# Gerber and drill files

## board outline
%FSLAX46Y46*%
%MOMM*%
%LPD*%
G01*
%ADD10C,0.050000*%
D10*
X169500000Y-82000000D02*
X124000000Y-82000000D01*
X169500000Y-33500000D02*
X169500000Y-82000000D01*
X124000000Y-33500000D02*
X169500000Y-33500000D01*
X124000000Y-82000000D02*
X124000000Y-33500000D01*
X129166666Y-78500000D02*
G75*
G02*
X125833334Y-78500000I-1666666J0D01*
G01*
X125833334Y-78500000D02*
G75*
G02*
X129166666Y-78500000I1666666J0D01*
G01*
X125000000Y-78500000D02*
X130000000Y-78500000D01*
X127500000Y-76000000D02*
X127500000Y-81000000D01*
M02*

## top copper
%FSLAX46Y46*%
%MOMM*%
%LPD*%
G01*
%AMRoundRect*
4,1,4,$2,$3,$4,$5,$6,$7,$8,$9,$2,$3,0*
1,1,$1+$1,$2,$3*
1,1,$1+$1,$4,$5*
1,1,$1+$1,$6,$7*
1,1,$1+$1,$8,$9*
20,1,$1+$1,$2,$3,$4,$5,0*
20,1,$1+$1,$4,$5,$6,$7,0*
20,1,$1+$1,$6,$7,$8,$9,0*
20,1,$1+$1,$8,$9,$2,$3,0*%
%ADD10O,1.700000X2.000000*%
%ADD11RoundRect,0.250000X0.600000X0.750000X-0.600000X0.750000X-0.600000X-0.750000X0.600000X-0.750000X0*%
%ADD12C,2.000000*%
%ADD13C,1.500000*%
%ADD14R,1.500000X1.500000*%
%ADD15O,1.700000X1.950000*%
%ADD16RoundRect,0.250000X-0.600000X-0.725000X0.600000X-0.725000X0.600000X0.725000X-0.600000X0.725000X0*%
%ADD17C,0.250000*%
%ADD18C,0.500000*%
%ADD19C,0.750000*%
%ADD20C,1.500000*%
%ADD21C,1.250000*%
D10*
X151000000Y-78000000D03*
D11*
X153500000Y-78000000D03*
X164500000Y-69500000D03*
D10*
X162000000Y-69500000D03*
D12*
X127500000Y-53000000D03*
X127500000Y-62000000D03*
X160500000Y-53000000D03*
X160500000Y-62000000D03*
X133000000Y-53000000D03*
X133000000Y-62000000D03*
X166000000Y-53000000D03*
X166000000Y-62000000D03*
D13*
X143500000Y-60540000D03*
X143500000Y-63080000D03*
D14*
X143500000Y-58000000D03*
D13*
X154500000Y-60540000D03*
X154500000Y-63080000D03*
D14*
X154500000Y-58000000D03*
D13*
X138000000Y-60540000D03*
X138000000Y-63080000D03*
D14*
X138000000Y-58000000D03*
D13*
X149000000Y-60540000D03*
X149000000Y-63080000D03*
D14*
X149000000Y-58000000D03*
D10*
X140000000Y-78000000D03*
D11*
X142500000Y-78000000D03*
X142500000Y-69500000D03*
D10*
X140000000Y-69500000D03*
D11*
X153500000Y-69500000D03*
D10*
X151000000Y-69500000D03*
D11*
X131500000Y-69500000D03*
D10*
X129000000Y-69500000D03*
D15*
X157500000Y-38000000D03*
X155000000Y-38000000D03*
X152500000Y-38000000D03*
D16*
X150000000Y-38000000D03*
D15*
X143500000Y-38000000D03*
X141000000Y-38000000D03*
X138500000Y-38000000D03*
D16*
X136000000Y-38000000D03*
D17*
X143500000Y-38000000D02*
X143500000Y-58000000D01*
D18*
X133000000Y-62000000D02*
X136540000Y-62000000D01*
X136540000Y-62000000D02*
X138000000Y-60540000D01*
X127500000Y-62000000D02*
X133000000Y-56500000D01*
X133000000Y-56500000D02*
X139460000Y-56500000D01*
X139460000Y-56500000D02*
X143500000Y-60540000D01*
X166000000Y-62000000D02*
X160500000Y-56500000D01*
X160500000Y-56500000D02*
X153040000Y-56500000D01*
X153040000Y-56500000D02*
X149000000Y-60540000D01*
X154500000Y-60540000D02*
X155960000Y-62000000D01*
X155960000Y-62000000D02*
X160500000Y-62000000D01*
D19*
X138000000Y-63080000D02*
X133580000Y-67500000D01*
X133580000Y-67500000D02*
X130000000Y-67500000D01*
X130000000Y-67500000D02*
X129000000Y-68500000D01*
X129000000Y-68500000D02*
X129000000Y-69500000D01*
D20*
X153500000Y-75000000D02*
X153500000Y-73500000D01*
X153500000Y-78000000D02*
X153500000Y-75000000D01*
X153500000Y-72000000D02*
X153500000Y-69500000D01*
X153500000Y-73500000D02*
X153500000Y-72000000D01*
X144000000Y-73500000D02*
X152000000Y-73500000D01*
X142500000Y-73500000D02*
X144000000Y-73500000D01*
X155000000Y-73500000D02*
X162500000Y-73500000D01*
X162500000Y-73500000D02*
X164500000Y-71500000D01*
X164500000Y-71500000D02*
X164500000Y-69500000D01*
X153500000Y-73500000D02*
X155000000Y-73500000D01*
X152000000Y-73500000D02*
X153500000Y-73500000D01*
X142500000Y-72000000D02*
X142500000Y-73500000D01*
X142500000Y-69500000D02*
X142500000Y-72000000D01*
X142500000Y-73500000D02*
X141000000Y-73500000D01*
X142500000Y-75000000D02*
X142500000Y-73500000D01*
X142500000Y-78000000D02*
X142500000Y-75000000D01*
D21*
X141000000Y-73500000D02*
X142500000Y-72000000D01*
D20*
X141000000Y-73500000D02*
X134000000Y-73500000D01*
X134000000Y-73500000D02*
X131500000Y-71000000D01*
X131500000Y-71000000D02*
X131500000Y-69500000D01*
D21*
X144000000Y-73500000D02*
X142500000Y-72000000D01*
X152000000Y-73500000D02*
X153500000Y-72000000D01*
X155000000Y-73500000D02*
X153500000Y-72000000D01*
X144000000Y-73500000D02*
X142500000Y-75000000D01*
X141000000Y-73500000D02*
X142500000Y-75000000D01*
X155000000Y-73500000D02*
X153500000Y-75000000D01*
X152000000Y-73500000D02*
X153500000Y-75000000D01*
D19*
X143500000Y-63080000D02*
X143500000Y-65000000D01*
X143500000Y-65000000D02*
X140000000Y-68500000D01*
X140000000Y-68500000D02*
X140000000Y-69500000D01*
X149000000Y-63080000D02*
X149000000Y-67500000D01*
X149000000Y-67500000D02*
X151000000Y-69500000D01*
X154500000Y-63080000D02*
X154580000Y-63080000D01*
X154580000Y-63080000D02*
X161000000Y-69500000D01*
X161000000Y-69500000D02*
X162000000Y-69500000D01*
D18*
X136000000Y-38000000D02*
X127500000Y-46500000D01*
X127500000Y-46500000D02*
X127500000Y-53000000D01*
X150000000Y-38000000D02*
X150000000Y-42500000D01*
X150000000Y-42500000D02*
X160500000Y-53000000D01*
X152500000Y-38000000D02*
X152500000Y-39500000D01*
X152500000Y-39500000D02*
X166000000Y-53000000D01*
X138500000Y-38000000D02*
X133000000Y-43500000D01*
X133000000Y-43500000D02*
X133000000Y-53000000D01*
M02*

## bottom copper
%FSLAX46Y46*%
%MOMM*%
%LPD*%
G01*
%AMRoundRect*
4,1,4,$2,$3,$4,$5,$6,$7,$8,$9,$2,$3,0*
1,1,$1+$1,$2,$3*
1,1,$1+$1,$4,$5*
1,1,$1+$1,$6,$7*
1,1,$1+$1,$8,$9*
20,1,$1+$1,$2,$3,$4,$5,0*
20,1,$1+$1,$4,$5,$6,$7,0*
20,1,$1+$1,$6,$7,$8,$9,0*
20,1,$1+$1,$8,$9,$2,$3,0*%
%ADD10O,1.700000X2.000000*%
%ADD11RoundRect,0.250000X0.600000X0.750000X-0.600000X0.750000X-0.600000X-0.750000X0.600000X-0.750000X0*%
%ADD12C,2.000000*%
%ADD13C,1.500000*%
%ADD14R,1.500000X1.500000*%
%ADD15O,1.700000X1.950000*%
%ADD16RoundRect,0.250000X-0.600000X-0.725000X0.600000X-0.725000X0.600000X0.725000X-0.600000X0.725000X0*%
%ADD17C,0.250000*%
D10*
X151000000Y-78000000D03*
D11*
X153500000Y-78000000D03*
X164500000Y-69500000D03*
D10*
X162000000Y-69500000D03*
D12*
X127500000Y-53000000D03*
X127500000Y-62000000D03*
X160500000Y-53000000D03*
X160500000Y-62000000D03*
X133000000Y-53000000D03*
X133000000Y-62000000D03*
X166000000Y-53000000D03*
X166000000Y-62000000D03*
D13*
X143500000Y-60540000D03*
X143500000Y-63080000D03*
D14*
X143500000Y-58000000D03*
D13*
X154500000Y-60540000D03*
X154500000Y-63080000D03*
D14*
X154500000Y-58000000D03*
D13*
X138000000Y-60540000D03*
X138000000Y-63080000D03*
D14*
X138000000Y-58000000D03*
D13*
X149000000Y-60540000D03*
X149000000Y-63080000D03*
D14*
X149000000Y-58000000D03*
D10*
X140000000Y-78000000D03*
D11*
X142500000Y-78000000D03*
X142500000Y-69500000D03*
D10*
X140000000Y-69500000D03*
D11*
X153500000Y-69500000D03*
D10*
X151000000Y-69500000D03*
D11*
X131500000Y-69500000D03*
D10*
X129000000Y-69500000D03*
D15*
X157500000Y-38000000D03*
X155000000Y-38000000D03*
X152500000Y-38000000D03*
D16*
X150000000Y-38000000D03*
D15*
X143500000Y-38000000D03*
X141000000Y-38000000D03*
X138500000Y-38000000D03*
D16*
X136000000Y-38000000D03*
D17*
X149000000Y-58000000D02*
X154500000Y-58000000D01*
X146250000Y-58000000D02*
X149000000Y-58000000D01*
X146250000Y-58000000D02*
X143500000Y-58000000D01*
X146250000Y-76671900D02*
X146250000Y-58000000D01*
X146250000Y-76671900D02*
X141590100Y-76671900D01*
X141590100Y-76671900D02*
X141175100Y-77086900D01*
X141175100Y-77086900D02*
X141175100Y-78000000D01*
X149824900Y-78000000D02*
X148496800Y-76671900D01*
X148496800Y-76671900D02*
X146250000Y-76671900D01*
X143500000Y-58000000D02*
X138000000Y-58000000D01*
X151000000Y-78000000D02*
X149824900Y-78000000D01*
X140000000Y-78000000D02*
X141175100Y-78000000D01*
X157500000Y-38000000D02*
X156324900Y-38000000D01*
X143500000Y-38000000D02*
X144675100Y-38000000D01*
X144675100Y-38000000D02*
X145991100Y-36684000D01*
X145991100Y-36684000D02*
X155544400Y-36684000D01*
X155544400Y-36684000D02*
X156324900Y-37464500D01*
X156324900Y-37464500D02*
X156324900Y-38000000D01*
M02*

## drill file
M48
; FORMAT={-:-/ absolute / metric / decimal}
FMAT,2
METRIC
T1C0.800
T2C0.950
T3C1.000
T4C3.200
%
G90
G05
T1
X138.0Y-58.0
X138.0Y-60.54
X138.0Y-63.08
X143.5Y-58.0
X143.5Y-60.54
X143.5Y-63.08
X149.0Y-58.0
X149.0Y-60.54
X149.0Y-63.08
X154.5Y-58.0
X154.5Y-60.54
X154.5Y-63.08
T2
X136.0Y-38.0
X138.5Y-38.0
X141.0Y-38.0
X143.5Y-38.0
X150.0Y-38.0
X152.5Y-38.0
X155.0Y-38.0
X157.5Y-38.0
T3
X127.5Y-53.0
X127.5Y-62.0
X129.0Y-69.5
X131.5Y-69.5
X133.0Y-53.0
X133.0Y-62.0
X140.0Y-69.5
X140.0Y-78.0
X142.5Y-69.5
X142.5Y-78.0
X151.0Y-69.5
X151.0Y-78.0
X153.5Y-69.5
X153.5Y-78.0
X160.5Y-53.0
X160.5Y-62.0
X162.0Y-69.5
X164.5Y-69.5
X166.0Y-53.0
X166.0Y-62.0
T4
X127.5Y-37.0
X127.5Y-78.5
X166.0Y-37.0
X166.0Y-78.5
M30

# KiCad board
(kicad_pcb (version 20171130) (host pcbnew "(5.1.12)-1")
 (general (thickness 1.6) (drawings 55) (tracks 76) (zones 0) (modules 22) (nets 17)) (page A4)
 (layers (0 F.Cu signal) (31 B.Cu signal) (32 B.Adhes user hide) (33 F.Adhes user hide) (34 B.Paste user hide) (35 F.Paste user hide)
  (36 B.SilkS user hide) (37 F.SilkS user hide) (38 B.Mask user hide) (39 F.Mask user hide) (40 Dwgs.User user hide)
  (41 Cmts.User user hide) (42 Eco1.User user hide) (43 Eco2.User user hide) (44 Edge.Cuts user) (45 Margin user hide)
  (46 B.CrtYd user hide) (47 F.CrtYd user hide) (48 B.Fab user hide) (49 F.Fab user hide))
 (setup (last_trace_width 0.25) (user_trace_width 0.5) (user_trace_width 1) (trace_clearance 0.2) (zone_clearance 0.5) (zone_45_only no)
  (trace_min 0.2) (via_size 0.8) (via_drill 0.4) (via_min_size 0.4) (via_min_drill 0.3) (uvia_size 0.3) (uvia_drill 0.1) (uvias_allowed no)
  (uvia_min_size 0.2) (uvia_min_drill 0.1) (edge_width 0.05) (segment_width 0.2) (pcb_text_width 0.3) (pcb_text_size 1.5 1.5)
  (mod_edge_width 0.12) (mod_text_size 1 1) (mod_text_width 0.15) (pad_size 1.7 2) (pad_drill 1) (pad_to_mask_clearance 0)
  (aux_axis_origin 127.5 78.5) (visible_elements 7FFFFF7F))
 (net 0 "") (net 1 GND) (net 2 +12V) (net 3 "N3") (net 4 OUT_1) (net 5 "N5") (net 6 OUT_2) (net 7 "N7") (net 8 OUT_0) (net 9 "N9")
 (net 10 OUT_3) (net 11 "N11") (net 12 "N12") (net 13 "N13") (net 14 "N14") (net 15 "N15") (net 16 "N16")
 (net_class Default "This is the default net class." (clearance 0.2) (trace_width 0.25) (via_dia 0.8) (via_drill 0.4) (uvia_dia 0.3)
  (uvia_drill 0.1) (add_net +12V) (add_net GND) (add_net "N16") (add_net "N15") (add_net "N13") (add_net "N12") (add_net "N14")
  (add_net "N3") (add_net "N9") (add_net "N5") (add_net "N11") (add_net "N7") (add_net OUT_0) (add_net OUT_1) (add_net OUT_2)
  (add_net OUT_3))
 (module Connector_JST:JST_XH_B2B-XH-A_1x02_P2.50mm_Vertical (layer F.Cu) (at 153.5 78 180)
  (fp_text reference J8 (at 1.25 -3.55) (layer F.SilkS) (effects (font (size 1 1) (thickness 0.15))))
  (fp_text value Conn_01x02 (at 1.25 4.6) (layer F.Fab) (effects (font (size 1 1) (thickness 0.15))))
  (pad 2 thru_hole oval (at 2.5 0 180) (size 1.7 2) (drill 1) (layers *.Cu *.Mask) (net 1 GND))
  (pad 1 thru_hole roundrect (at 0 0 180) (size 1.7 2) (drill 1) (layers *.Cu *.Mask) (roundrect_rratio 0.1470588235294118) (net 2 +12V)))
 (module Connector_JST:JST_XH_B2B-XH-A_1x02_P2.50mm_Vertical (layer F.Cu) (at 164.5 69.5 180)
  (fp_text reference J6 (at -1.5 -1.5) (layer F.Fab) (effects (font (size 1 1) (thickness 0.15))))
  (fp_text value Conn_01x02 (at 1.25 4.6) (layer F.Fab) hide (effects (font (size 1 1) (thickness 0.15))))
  (pad 1 thru_hole roundrect (at 0 0 180) (size 1.7 2) (drill 1) (layers *.Cu *.Mask) (roundrect_rratio 0.1470588235294118) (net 2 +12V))
  (pad 2 thru_hole oval (at 2.5 0 180) (size 1.7 2) (drill 1) (layers *.Cu *.Mask) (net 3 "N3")))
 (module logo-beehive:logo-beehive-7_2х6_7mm (layer F.Cu) (at 133 77 90)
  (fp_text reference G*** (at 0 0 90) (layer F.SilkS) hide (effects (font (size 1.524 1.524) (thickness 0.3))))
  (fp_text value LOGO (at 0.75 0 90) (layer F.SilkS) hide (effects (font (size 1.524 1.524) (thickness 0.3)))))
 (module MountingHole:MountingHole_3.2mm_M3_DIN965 (layer F.Cu) (at 166 37 270)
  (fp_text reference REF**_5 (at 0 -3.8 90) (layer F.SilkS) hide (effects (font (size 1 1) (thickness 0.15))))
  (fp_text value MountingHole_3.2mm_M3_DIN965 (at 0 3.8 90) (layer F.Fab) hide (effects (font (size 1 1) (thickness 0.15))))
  (pad 1 np_thru_hole circle (at 0 0 270) (size 3.2 3.2) (drill 3.2) (layers *.Cu *.Mask)))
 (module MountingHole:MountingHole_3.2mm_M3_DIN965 (layer F.Cu) (at 166 78.5 180)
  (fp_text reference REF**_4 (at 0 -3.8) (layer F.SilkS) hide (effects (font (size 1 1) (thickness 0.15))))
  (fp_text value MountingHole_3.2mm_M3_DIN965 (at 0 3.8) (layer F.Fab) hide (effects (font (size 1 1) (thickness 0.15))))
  (pad 1 np_thru_hole circle (at 0 0 180) (size 3.2 3.2) (drill 3.2) (layers *.Cu *.Mask)))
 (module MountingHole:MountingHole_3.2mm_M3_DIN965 (layer F.Cu) (at 127.5 78.5 90)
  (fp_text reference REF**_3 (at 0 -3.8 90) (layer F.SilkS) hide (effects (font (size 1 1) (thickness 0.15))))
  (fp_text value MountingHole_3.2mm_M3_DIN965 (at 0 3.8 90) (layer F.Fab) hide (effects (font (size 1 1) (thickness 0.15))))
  (pad 1 np_thru_hole circle (at 0 0 90) (size 3.2 3.2) (drill 3.2) (layers *.Cu *.Mask)))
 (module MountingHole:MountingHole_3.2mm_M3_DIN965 (layer F.Cu) (at 127.5 37 90)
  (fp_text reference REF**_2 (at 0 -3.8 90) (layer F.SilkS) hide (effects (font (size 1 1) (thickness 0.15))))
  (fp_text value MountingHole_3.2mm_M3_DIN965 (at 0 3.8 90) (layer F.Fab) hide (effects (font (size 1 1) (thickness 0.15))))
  (pad 1 np_thru_hole circle (at 0 0 90) (size 3.2 3.2) (drill 3.2) (layers *.Cu *.Mask)))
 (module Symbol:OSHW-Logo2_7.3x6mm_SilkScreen (layer F.Cu) (at 147 51)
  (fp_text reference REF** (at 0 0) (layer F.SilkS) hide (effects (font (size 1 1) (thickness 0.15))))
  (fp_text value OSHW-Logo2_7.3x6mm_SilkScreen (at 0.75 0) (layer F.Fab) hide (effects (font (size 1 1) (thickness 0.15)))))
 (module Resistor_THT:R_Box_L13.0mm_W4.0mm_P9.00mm (layer F.Cu) (at 127.5 53 270)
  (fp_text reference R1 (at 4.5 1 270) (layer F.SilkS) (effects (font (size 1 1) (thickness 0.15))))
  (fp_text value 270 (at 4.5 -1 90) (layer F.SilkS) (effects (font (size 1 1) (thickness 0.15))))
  (pad 1 thru_hole circle (at 0 0 270) (size 2 2) (drill 1) (layers *.Cu *.Mask) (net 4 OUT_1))
  (pad 2 thru_hole circle (at 9 0 270) (size 2 2) (drill 1) (layers *.Cu *.Mask) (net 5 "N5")))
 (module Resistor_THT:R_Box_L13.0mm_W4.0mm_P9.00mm (layer F.Cu) (at 160.5 53 270)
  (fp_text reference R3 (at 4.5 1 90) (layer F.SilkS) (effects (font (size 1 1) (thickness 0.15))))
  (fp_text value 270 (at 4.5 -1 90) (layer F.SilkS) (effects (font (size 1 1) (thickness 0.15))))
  (pad 1 thru_hole circle (at 0 0 270) (size 2 2) (drill 1) (layers *.Cu *.Mask) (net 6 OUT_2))
  (pad 2 thru_hole circle (at 9 0 270) (size 2 2) (drill 1) (layers *.Cu *.Mask) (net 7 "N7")))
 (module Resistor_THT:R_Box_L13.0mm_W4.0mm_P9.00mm (layer F.Cu) (at 133 53 270)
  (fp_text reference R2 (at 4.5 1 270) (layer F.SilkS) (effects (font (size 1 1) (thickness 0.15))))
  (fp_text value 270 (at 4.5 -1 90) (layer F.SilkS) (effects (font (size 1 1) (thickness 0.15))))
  (pad 1 thru_hole circle (at 0 0 270) (size 2 2) (drill 1) (layers *.Cu *.Mask) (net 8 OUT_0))
  (pad 2 thru_hole circle (at 9 0 270) (size 2 2) (drill 1) (layers *.Cu *.Mask) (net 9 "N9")))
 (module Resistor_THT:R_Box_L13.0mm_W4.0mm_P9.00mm (layer F.Cu) (at 166 53 270)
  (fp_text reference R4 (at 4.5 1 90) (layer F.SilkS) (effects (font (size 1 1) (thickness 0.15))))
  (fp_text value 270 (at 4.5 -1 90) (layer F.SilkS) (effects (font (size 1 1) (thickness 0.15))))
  (pad 1 thru_hole circle (at 0 0 270) (size 2 2) (drill 1) (layers *.Cu *.Mask) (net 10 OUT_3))
  (pad 2 thru_hole circle (at 9 0 270) (size 2 2) (drill 1) (layers *.Cu *.Mask) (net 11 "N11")))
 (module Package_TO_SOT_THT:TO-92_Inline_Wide (layer F.Cu) (at 143.5 58 270)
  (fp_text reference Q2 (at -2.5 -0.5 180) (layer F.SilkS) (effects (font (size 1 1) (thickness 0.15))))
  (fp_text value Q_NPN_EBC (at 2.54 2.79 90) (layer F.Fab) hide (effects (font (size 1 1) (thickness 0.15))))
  (pad 2 thru_hole circle (at 2.54 0) (size 1.5 1.5) (drill 0.8) (layers *.Cu *.Mask) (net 5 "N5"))
  (pad 3 thru_hole circle (at 5.08 0) (size 1.5 1.5) (drill 0.8) (layers *.Cu *.Mask) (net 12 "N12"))
  (pad 1 thru_hole rect (at 0 0) (size 1.5 1.5) (drill 0.8) (layers *.Cu *.Mask) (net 1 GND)))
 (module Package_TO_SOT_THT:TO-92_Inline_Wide (layer F.Cu) (at 154.5 58 270)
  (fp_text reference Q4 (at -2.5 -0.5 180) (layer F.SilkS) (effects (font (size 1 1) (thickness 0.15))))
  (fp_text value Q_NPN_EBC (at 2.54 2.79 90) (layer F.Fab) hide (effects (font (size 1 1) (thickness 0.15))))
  (pad 2 thru_hole circle (at 2.54 0) (size 1.5 1.5) (drill 0.8) (layers *.Cu *.Mask) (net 7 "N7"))
  (pad 3 thru_hole circle (at 5.08 0) (size 1.5 1.5) (drill 0.8) (layers *.Cu *.Mask) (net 3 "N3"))
  (pad 1 thru_hole rect (at 0 0) (size 1.5 1.5) (drill 0.8) (layers *.Cu *.Mask) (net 1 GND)))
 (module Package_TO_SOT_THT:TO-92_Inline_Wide (layer F.Cu) (at 138 58 270)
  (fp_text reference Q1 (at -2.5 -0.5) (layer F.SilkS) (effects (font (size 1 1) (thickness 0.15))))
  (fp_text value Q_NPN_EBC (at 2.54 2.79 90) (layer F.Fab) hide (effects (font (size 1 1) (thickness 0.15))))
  (pad 2 thru_hole circle (at 2.54 0) (size 1.5 1.5) (drill 0.8) (layers *.Cu *.Mask) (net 9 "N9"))
  (pad 3 thru_hole circle (at 5.08 0) (size 1.5 1.5) (drill 0.8) (layers *.Cu *.Mask) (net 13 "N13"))
  (pad 1 thru_hole rect (at 0 0) (size 1.5 1.5) (drill 0.8) (layers *.Cu *.Mask) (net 1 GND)))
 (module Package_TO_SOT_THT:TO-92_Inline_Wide (layer F.Cu) (at 149 58 270)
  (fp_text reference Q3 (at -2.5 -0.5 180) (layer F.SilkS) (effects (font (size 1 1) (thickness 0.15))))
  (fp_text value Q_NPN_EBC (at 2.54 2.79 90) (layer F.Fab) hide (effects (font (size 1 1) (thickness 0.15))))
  (pad 2 thru_hole circle (at 2.54 0) (size 1.5 1.5) (drill 0.8) (layers *.Cu *.Mask) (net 11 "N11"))
  (pad 3 thru_hole circle (at 5.08 0) (size 1.5 1.5) (drill 0.8) (layers *.Cu *.Mask) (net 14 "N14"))
  (pad 1 thru_hole rect (at 0 0) (size 1.5 1.5) (drill 0.8) (layers *.Cu *.Mask) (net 1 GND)))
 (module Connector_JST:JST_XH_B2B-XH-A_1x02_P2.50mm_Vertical (layer F.Cu) (at 142.5 78 180)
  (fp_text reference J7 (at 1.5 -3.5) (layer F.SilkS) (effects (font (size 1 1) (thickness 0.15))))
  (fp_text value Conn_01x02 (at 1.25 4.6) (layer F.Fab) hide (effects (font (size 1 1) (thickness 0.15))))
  (pad 2 thru_hole oval (at 2.5 0 180) (size 1.7 2) (drill 1) (layers *.Cu *.Mask) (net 1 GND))
  (pad 1 thru_hole roundrect (at 0 0 180) (size 1.7 2) (drill 1) (layers *.Cu *.Mask) (roundrect_rratio 0.1470588235294118) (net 2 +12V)))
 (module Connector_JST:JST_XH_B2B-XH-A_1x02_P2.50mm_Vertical (layer F.Cu) (at 142.5 69.5 180)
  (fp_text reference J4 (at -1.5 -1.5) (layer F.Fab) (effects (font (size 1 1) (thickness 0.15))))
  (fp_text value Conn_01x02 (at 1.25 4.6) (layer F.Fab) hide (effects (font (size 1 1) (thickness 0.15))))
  (pad 1 thru_hole roundrect (at 0 0 180) (size 1.7 2) (drill 1) (layers *.Cu *.Mask) (roundrect_rratio 0.1470588235294118) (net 2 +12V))
  (pad 2 thru_hole oval (at 2.5 0 180) (size 1.7 2) (drill 1) (layers *.Cu *.Mask) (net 12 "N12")))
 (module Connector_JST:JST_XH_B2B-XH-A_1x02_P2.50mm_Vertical (layer F.Cu) (at 153.5 69.5 180)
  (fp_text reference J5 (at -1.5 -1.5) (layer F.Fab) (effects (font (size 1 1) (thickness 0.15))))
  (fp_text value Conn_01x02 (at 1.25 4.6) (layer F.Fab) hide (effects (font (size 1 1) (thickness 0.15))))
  (pad 1 thru_hole roundrect (at 0 0 180) (size 1.7 2) (drill 1) (layers *.Cu *.Mask) (roundrect_rratio 0.1470588235294118) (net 2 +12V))
  (pad 2 thru_hole oval (at 2.5 0 180) (size 1.7 2) (drill 1) (layers *.Cu *.Mask) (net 14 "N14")))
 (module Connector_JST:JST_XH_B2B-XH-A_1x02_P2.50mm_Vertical (layer F.Cu) (at 131.5 69.5 180)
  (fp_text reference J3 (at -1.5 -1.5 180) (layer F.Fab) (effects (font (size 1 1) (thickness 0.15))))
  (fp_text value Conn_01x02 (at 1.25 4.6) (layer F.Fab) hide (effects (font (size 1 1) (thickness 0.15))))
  (pad 1 thru_hole roundrect (at 0 0 180) (size 1.7 2) (drill 1) (layers *.Cu *.Mask) (roundrect_rratio 0.1470588235294118) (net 2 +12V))
  (pad 2 thru_hole oval (at 2.5 0 180) (size 1.7 2) (drill 1) (layers *.Cu *.Mask) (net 13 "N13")))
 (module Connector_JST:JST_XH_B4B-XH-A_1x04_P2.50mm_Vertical (layer F.Cu) (at 150 38)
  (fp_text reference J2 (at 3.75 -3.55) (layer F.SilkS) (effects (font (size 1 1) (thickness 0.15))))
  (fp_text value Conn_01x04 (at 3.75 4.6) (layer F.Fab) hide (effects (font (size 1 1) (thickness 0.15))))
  (pad 4 thru_hole oval (at 7.5 0) (size 1.7 1.95) (drill 0.95) (layers *.Cu *.Mask) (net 1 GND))
  (pad 3 thru_hole oval (at 5 0) (size 1.7 1.95) (drill 0.95) (layers *.Cu *.Mask) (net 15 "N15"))
  (pad 2 thru_hole oval (at 2.5 0) (size 1.7 1.95) (drill 0.95) (layers *.Cu *.Mask) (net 10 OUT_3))
  (pad 1 thru_hole roundrect (at 0 0) (size 1.7 1.95) (drill 0.95) (layers *.Cu *.Mask) (roundrect_rratio 0.1470588235294118) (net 6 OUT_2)))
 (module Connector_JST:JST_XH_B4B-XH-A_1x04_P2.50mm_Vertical (layer F.Cu) (at 136 38)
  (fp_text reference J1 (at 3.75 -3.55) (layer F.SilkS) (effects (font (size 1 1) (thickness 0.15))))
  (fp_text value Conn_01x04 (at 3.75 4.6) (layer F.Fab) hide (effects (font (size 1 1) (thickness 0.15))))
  (pad 4 thru_hole oval (at 7.5 0) (size 1.7 1.95) (drill 0.95) (layers *.Cu *.Mask) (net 1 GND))
  (pad 3 thru_hole oval (at 5 0) (size 1.7 1.95) (drill 0.95) (layers *.Cu *.Mask) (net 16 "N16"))
  (pad 2 thru_hole oval (at 2.5 0) (size 1.7 1.95) (drill 0.95) (layers *.Cu *.Mask) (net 8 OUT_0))
  (pad 1 thru_hole roundrect (at 0 0) (size 1.7 1.95) (drill 0.95) (layers *.Cu *.Mask) (roundrect_rratio 0.1470588235294118) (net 4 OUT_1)))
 (gr_line (start 169.5 82) (end 124 82) (layer Edge.Cuts) (width 0.05))
 (gr_line (start 169.5 33.5) (end 169.5 82) (layer Edge.Cuts) (width 0.05))
 (gr_line (start 124 33.5) (end 169.5 33.5) (layer Edge.Cuts) (width 0.05))
 (gr_line (start 124 82) (end 124 33.5) (layer Edge.Cuts) (width 0.05))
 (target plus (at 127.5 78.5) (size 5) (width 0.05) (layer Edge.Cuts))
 (segment (start 149 58) (end 154.5 58) (width 0.25) (layer B.Cu) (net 1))
 (segment (start 146.25 58) (end 149 58) (width 0.25) (layer B.Cu) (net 1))
 (segment (start 146.25 58) (end 143.5 58) (width 0.25) (layer B.Cu) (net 1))
 (segment (start 146.25 76.6719) (end 146.25 58) (width 0.25) (layer B.Cu) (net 1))
 (segment (start 146.25 76.6719) (end 141.5901 76.6719) (width 0.25) (layer B.Cu) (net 1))
 (segment (start 141.5901 76.6719) (end 141.1751 77.0869) (width 0.25) (layer B.Cu) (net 1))
 (segment (start 141.1751 77.0869) (end 141.1751 78) (width 0.25) (layer B.Cu) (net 1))
 (segment (start 149.8249 78) (end 148.4968 76.6719) (width 0.25) (layer B.Cu) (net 1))
 (segment (start 148.4968 76.6719) (end 146.25 76.6719) (width 0.25) (layer B.Cu) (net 1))
 (segment (start 143.5 58) (end 138 58) (width 0.25) (layer B.Cu) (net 1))
 (segment (start 151 78) (end 149.8249 78) (width 0.25) (layer B.Cu) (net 1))
 (segment (start 140 78) (end 141.1751 78) (width 0.25) (layer B.Cu) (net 1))
 (segment (start 143.5 38) (end 143.5 58) (width 0.25) (layer F.Cu) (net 1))
 (segment (start 157.5 38) (end 156.3249 38) (width 0.25) (layer B.Cu) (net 1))
 (segment (start 143.5 38) (end 144.6751 38) (width 0.25) (layer B.Cu) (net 1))
 (segment (start 144.6751 38) (end 145.9911 36.684) (width 0.25) (layer B.Cu) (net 1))
 (segment (start 145.9911 36.684) (end 155.5444 36.684) (width 0.25) (layer B.Cu) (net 1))
 (segment (start 155.5444 36.684) (end 156.3249 37.4645) (width 0.25) (layer B.Cu) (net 1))
 (segment (start 156.3249 37.4645) (end 156.3249 38) (width 0.25) (layer B.Cu) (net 1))
 (segment (start 133 62) (end 136.54 62) (width 0.5) (layer F.Cu) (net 9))
 (segment (start 136.54 62) (end 138 60.54) (width 0.5) (layer F.Cu) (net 9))
 (segment (start 127.5 62) (end 133 56.5) (width 0.5) (layer F.Cu) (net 5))
 (segment (start 133 56.5) (end 139.46 56.5) (width 0.5) (layer F.Cu) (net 5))
 (segment (start 139.46 56.5) (end 143.5 60.54) (width 0.5) (layer F.Cu) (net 5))
 (segment (start 166 62) (end 160.5 56.5) (width 0.5) (layer F.Cu) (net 11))
 (segment (start 160.5 56.5) (end 153.04 56.5) (width 0.5) (layer F.Cu) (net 11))
 (segment (start 153.04 56.5) (end 149 60.54) (width 0.5) (layer F.Cu) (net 11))
 (segment (start 154.5 60.54) (end 155.96 62) (width 0.5) (layer F.Cu) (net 7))
 (segment (start 155.96 62) (end 160.5 62) (width 0.5) (layer F.Cu) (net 7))
 (segment (start 138 63.08) (end 133.58 67.5) (width 0.75) (layer F.Cu) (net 13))
 (segment (start 133.58 67.5) (end 130 67.5) (width 0.75) (layer F.Cu) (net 13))
 (segment (start 130 67.5) (end 129 68.5) (width 0.75) (layer F.Cu) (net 13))
 (segment (start 129 68.5) (end 129 69.5) (width 0.75) (layer F.Cu) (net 13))
 (segment (start 153.5 75) (end 153.5 73.5) (width 1.5) (layer F.Cu) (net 2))
 (segment (start 153.5 78) (end 153.5 75) (width 1.5) (layer F.Cu) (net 2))
 (segment (start 153.5 72) (end 153.5 69.5) (width 1.5) (layer F.Cu) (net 2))
 (segment (start 153.5 73.5) (end 153.5 72) (width 1.5) (layer F.Cu) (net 2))
 (segment (start 144 73.5) (end 152 73.5) (width 1.5) (layer F.Cu) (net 2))
 (segment (start 142.5 73.5) (end 144 73.5) (width 1.5) (layer F.Cu) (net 2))
 (segment (start 155 73.5) (end 162.5 73.5) (width 1.5) (layer F.Cu) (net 2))
 (segment (start 162.5 73.5) (end 164.5 71.5) (width 1.5) (layer F.Cu) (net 2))
 (segment (start 164.5 71.5) (end 164.5 69.5) (width 1.5) (layer F.Cu) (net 2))
 (segment (start 153.5 73.5) (end 155 73.5) (width 1.5) (layer F.Cu) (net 2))
 (segment (start 152 73.5) (end 153.5 73.5) (width 1.5) (layer F.Cu) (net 2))
 (segment (start 142.5 72) (end 142.5 73.5) (width 1.5) (layer F.Cu) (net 2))
 (segment (start 142.5 69.5) (end 142.5 72) (width 1.5) (layer F.Cu) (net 2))
 (segment (start 142.5 73.5) (end 141 73.5) (width 1.5) (layer F.Cu) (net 2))
 (segment (start 142.5 75) (end 142.5 73.5) (width 1.5) (layer F.Cu) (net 2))
 (segment (start 142.5 78) (end 142.5 75) (width 1.5) (layer F.Cu) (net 2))
 (segment (start 141 73.5) (end 142.5 72) (width 1.25) (layer F.Cu) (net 2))
 (segment (start 141 73.5) (end 134 73.5) (width 1.5) (layer F.Cu) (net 2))
 (segment (start 134 73.5) (end 131.5 71) (width 1.5) (layer F.Cu) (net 2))
 (segment (start 131.5 71) (end 131.5 69.5) (width 1.5) (layer F.Cu) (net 2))
 (segment (start 144 73.5) (end 142.5 72) (width 1.25) (layer F.Cu) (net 2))
 (segment (start 152 73.5) (end 153.5 72) (width 1.25) (layer F.Cu) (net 2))
 (segment (start 155 73.5) (end 153.5 72) (width 1.25) (layer F.Cu) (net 2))
 (segment (start 144 73.5) (end 142.5 75) (width 1.25) (layer F.Cu) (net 2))
 (segment (start 141 73.5) (end 142.5 75) (width 1.25) (layer F.Cu) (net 2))
 (segment (start 155 73.5) (end 153.5 75) (width 1.25) (layer F.Cu) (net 2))
 (segment (start 152 73.5) (end 153.5 75) (width 1.25) (layer F.Cu) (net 2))
 (segment (start 143.5 63.08) (end 143.5 65) (width 0.75) (layer F.Cu) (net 12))
 (segment (start 143.5 65) (end 140 68.5) (width 0.75) (layer F.Cu) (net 12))
 (segment (start 140 68.5) (end 140 69.5) (width 0.75) (layer F.Cu) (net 12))
 (segment (start 149 63.08) (end 149 67.5) (width 0.75) (layer F.Cu) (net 14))
 (segment (start 149 67.5) (end 151 69.5) (width 0.75) (layer F.Cu) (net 14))
 (segment (start 154.5 63.08) (end 154.58 63.08) (width 0.75) (layer F.Cu) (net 3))
 (segment (start 154.58 63.08) (end 161 69.5) (width 0.75) (layer F.Cu) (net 3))
 (segment (start 161 69.5) (end 162 69.5) (width 0.75) (layer F.Cu) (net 3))
 (segment (start 136 38) (end 127.5 46.5) (width 0.5) (layer F.Cu) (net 4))
 (segment (start 127.5 46.5) (end 127.5 53) (width 0.5) (layer F.Cu) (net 4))
 (segment (start 150 38) (end 150 42.5) (width 0.5) (layer F.Cu) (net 6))
 (segment (start 150 42.5) (end 160.5 53) (width 0.5) (layer F.Cu) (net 6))
 (segment (start 152.5 38) (end 152.5 39.5) (width 0.5) (layer F.Cu) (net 10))
 (segment (start 152.5 39.5) (end 166 53) (width 0.5) (layer F.Cu) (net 10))
 (segment (start 138.5 38) (end 133 43.5) (width 0.5) (layer F.Cu) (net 8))
 (segment (start 133 43.5) (end 133 53) (width 0.5) (layer F.Cu) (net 8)))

